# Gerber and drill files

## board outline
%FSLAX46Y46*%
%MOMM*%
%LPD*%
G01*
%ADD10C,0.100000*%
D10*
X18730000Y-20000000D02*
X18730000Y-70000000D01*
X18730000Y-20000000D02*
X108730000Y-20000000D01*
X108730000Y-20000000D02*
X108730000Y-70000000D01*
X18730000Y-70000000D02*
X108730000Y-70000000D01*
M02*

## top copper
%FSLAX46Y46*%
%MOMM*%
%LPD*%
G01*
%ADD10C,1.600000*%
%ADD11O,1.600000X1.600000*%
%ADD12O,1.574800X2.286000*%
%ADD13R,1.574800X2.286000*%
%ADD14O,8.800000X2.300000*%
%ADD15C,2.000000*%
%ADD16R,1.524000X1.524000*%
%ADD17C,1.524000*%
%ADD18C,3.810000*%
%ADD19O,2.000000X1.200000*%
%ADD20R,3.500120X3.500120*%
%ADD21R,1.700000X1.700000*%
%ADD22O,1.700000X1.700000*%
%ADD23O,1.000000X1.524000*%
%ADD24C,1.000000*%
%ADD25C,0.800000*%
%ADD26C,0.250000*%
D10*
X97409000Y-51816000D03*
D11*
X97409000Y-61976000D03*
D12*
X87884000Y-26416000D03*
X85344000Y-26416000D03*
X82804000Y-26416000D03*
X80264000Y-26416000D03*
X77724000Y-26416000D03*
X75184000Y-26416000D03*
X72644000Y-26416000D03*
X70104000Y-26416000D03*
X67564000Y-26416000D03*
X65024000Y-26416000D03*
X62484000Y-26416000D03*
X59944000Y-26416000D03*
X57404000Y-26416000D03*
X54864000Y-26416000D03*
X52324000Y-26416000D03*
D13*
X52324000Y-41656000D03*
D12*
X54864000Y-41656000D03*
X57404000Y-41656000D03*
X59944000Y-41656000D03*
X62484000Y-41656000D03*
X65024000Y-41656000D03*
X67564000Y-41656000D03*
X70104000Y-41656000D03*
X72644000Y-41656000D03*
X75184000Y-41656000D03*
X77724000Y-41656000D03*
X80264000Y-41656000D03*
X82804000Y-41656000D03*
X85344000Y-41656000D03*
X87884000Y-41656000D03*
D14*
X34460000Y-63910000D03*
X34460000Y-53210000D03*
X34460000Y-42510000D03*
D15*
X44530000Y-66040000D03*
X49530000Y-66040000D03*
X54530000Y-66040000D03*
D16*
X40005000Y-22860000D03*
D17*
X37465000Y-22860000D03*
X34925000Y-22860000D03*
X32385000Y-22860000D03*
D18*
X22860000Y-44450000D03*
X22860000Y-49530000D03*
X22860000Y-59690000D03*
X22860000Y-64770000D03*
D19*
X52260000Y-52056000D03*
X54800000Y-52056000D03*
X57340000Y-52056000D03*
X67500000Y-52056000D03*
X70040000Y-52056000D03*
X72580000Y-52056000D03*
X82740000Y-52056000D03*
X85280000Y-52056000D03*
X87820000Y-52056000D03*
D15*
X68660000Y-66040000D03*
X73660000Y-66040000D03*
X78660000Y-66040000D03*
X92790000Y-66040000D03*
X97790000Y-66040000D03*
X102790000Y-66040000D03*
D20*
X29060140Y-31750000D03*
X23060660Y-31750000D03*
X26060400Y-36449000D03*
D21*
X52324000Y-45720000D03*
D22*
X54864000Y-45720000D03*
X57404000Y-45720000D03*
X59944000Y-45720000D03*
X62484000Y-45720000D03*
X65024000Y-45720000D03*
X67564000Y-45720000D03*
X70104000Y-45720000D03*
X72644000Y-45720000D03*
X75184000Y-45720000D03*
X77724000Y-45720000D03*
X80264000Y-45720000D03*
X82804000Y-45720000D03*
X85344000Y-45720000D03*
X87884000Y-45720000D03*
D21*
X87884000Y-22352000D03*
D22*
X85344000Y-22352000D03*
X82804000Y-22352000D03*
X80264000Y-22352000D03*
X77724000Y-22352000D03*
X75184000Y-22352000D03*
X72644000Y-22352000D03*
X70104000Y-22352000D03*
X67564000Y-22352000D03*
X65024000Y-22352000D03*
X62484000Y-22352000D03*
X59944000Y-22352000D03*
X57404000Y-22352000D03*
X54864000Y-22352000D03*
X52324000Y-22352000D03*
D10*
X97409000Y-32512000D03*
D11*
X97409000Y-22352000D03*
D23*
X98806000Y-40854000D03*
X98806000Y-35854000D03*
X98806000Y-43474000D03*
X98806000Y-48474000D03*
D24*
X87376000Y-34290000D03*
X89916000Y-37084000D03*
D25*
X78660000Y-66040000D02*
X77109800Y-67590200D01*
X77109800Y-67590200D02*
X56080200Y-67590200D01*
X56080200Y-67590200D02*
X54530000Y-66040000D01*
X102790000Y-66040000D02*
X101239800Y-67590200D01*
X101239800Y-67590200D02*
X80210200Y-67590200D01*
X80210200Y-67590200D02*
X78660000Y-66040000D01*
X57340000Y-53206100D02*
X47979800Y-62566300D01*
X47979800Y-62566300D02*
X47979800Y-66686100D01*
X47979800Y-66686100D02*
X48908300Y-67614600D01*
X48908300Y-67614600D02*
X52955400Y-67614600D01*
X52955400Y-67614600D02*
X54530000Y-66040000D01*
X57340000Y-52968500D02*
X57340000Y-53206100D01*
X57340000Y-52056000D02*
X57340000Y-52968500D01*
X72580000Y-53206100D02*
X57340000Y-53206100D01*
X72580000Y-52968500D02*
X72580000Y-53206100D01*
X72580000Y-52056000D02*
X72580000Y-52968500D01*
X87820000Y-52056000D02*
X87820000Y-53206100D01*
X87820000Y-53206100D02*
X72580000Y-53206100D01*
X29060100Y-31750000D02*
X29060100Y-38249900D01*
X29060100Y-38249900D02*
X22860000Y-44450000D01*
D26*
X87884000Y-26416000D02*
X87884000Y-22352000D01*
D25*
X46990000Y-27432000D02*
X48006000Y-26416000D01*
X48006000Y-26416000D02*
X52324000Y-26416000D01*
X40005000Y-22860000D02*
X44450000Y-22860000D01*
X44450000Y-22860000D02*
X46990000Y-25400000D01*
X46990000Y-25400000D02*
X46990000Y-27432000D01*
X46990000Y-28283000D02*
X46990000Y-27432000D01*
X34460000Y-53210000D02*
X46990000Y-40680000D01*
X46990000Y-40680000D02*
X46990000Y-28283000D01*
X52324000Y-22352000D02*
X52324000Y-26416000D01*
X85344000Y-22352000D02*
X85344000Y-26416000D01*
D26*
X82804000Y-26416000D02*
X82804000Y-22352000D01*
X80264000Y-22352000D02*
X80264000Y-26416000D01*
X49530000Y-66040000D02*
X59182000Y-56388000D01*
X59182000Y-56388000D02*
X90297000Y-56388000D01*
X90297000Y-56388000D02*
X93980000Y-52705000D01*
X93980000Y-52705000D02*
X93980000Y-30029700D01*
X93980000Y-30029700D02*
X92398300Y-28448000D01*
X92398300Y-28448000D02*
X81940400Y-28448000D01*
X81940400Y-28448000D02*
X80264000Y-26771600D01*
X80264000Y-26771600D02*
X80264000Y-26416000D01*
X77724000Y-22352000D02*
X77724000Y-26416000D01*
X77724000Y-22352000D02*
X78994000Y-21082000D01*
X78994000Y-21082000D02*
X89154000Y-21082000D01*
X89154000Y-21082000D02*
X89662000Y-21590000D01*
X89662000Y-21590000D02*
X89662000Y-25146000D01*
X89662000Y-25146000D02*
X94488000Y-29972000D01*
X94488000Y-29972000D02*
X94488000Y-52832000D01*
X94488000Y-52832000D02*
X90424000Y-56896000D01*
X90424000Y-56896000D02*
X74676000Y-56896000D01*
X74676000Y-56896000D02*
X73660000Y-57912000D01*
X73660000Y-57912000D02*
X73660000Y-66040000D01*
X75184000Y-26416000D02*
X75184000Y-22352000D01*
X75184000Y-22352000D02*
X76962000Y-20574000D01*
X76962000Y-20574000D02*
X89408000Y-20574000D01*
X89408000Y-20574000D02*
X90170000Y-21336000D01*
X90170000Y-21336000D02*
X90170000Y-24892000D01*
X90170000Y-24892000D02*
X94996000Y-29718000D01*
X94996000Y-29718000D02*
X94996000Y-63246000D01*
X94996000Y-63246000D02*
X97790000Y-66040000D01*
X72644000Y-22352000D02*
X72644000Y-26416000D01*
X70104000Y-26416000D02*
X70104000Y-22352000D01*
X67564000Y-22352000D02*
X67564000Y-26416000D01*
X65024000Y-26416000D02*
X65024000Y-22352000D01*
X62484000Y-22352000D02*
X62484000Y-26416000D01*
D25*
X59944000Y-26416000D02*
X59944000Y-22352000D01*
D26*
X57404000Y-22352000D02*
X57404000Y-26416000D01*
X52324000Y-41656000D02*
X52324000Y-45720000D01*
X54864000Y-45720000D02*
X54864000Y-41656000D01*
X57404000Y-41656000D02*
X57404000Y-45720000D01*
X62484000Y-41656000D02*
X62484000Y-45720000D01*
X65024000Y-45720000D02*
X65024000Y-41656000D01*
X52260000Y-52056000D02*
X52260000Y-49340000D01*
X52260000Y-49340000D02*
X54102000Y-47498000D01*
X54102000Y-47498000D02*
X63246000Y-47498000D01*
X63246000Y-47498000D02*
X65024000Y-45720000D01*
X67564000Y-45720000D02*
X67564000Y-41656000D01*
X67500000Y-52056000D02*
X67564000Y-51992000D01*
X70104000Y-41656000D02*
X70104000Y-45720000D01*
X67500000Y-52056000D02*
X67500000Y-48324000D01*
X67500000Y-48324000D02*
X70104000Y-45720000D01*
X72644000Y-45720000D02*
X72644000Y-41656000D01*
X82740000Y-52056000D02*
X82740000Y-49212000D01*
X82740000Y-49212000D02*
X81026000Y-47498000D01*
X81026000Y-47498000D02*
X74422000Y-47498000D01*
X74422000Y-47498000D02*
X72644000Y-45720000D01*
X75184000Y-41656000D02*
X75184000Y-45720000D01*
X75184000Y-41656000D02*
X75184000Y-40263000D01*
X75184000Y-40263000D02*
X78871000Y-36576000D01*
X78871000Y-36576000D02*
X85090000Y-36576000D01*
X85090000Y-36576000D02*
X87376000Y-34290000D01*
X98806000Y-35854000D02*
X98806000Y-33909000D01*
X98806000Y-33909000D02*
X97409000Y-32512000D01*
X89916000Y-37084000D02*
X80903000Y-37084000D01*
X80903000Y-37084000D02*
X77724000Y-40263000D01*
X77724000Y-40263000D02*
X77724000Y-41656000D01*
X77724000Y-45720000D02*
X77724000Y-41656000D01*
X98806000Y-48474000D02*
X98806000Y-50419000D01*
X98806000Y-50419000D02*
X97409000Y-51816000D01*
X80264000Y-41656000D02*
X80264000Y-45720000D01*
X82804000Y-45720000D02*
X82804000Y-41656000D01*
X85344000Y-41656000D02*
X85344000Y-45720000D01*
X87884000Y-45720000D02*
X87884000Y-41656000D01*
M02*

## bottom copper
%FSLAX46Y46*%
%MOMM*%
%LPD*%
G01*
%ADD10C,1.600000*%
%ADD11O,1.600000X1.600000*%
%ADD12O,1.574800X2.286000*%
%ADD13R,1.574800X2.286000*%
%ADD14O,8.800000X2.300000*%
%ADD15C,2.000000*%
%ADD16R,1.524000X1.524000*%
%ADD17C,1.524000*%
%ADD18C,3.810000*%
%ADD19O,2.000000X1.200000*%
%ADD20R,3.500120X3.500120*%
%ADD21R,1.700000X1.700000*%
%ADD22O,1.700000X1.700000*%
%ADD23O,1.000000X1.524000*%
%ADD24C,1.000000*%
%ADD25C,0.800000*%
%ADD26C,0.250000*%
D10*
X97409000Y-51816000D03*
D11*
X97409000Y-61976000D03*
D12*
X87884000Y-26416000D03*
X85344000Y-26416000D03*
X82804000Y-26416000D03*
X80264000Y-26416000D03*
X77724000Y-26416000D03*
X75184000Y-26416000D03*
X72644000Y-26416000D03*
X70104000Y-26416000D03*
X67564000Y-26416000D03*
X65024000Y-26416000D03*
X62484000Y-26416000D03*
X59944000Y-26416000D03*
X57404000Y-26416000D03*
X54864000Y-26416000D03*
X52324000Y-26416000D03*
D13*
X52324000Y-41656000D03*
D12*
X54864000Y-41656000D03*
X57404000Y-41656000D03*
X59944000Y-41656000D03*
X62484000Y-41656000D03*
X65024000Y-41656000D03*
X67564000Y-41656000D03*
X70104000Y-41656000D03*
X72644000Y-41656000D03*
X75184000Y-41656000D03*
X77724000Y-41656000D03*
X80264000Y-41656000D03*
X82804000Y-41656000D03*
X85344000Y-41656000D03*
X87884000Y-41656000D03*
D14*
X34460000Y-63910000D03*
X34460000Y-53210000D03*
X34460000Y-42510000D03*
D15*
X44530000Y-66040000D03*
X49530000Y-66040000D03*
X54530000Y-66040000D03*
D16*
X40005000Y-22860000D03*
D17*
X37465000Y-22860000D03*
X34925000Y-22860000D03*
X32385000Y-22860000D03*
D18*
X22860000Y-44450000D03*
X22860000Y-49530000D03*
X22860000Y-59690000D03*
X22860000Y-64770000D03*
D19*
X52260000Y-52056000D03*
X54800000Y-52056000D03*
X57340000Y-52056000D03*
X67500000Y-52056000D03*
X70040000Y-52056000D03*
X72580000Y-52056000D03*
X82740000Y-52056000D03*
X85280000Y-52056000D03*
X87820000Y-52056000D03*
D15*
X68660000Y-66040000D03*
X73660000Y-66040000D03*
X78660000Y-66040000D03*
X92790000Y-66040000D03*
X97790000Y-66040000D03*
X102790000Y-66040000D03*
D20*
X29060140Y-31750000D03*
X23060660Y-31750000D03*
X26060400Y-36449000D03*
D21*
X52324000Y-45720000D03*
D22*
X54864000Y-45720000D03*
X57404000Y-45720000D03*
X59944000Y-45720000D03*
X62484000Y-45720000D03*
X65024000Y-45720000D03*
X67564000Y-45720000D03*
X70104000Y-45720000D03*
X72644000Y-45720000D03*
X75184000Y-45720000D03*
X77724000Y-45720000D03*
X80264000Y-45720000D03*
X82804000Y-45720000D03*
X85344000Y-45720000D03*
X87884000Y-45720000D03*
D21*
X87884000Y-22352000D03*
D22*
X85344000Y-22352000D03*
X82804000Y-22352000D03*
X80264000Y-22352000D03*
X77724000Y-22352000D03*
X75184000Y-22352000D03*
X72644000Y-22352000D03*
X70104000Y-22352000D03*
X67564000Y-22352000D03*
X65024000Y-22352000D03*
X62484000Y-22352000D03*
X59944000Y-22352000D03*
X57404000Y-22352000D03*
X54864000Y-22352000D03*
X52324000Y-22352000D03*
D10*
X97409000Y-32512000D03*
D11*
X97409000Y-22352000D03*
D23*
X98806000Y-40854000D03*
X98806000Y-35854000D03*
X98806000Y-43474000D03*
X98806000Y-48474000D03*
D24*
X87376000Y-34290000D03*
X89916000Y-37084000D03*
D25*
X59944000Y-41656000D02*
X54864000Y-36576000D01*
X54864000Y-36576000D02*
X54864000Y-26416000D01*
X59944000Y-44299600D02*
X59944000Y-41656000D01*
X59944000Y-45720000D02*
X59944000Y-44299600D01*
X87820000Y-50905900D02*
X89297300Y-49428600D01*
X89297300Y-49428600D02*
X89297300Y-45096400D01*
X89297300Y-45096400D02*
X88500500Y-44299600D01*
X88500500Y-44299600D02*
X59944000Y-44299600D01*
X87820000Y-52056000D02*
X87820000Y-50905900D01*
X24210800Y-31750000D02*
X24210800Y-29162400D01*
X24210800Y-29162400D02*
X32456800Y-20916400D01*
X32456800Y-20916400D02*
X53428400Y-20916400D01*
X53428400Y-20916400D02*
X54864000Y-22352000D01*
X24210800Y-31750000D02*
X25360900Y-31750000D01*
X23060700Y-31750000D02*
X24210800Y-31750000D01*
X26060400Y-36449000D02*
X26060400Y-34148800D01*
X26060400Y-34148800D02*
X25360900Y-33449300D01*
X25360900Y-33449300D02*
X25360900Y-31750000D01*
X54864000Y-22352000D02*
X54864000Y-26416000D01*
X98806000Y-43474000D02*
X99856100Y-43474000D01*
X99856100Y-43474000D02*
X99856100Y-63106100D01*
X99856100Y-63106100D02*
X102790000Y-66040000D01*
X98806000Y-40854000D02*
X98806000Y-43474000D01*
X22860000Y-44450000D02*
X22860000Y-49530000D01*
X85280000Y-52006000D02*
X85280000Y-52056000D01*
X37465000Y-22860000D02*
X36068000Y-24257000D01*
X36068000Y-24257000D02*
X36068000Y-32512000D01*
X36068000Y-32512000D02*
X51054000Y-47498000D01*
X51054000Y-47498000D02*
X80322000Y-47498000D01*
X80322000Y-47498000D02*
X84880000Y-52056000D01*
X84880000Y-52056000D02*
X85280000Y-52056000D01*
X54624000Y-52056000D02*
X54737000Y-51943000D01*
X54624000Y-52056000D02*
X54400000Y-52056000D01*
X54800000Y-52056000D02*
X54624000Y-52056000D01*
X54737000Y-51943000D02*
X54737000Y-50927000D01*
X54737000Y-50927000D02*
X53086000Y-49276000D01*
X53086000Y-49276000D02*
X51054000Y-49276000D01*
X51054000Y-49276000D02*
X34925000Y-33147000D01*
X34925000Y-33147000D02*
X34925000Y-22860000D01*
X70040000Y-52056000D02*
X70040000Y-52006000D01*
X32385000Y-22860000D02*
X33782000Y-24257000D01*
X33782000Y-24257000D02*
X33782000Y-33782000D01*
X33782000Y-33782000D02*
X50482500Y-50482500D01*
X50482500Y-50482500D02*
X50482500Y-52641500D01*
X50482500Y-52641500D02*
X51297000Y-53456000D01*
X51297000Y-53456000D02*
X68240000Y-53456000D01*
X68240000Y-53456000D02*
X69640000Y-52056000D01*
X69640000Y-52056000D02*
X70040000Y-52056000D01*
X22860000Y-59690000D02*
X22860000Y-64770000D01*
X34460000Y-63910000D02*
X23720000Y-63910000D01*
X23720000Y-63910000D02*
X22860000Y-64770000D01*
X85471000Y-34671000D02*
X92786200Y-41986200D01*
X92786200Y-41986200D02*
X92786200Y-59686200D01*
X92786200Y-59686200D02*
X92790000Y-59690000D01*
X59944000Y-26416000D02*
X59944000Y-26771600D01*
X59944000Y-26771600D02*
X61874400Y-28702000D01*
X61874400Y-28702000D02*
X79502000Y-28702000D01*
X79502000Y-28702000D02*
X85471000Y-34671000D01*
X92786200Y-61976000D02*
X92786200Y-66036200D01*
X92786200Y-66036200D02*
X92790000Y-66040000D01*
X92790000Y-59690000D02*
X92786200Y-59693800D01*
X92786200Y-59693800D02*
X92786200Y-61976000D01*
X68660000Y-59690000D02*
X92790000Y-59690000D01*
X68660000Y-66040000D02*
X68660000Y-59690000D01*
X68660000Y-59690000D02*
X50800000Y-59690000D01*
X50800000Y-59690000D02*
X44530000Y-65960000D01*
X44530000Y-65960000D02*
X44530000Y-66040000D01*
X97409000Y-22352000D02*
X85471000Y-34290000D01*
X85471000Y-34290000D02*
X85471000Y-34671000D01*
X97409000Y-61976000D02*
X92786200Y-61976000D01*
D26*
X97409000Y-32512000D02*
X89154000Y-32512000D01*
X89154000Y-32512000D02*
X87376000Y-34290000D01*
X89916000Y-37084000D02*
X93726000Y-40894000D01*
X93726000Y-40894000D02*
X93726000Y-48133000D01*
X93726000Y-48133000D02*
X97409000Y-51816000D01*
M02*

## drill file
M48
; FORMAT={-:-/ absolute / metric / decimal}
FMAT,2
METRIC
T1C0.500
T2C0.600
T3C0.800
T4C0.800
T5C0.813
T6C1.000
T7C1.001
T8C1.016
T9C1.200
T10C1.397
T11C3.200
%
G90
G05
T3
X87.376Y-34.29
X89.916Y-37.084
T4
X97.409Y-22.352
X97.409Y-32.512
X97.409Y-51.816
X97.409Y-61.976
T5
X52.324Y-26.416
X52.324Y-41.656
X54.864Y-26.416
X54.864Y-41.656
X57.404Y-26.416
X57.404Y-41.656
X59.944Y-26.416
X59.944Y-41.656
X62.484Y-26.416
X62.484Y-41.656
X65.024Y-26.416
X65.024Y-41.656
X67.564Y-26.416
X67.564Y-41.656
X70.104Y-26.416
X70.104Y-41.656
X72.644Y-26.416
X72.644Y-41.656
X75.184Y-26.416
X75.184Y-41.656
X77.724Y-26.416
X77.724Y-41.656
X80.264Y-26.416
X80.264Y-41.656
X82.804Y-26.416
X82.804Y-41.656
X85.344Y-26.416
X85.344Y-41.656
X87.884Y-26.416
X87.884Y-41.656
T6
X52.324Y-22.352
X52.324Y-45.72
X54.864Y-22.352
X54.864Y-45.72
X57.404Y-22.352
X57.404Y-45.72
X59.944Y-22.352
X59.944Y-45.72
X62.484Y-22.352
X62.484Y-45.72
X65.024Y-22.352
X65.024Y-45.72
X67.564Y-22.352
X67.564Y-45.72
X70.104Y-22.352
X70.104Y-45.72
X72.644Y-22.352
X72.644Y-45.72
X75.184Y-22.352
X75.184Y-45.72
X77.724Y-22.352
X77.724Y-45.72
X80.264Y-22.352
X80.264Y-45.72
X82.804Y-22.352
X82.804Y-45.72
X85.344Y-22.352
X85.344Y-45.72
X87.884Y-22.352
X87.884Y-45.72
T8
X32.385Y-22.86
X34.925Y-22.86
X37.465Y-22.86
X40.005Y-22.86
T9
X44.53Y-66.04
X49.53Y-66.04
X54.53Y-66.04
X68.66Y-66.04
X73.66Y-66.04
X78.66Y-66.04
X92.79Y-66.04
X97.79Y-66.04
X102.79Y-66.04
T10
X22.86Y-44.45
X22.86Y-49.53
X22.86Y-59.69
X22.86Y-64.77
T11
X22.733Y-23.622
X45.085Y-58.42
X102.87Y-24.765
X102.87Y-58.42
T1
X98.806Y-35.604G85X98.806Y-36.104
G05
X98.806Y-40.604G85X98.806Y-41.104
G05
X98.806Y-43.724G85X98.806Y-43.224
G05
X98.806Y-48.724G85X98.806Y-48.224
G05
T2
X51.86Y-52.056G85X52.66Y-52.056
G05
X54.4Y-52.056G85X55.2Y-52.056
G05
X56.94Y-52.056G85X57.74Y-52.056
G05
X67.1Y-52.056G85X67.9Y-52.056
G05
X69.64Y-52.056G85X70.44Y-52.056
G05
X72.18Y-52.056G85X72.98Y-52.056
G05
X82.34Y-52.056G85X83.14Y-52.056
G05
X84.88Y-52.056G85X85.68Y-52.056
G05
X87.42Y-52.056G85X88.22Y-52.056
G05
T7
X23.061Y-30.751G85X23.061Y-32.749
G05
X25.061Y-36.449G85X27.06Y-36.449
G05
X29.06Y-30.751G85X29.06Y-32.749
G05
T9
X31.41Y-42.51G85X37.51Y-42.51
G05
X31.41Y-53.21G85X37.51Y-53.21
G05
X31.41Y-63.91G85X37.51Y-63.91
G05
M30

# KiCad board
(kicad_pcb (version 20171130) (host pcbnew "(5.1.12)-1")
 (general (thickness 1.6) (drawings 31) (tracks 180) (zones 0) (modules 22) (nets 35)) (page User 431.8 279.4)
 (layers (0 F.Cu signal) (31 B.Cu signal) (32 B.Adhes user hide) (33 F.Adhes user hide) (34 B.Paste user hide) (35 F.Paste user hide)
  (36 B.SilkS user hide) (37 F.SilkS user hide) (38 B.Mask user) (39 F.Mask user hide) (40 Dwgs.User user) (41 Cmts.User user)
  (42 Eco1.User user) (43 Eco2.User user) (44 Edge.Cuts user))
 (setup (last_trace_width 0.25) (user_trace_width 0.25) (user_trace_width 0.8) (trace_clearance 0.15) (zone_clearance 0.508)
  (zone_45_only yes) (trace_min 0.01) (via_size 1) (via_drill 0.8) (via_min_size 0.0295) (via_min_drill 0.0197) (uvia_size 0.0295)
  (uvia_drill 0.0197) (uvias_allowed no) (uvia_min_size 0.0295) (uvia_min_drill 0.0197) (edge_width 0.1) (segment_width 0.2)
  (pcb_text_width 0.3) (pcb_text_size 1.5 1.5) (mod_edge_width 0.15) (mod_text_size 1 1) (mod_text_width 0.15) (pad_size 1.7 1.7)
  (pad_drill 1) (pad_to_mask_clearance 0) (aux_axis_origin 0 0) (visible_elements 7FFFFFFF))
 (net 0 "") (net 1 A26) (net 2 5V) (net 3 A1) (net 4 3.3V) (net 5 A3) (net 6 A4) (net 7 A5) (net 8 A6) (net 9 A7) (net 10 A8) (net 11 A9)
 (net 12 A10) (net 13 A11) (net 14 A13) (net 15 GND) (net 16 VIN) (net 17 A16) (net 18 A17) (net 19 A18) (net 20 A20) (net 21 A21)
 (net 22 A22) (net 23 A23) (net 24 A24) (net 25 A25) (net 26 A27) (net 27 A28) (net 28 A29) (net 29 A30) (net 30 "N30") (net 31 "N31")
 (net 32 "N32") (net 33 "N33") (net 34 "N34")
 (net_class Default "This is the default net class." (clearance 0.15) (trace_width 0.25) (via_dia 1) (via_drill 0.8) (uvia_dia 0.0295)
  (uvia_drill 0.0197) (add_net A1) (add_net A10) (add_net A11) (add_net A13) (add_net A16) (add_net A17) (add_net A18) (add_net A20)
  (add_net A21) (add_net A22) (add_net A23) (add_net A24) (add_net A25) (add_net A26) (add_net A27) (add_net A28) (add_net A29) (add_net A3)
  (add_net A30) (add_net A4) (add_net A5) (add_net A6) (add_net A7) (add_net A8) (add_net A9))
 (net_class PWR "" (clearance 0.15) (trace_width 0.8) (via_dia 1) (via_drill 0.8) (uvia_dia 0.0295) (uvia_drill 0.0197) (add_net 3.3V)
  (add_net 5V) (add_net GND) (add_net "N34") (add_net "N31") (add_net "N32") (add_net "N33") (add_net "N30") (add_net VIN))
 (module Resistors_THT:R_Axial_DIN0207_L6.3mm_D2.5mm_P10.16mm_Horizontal (layer F.Cu) (at 97.409 51.816 270)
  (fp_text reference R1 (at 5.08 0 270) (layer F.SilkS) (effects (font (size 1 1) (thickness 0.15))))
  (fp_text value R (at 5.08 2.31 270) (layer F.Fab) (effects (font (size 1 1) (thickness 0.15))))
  (pad 1 thru_hole circle (at 0 0 270) (size 1.6 1.6) (drill 0.8) (layers *.Cu *.Mask) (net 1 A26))
  (pad 2 thru_hole oval (at 10.16 0 270) (size 1.6 1.6) (drill 0.8) (layers *.Cu *.Mask) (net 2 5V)))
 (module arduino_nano (layer F.Cu) (at 68.834 34.036 180)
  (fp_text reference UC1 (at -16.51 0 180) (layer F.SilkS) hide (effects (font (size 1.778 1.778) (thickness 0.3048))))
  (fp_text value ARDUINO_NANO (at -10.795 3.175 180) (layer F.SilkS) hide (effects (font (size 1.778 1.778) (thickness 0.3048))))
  (pad 1 thru_hole oval (at -19.05 7.62 180) (size 1.5748 2.286) (drill 0.8128) (layers *.Cu *.Mask F.SilkS) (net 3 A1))
  (pad 2 thru_hole oval (at -16.51 7.62 180) (size 1.5748 2.286) (drill 0.8128) (layers *.Cu *.Mask F.SilkS) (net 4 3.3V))
  (pad 3 thru_hole oval (at -13.97 7.62 180) (size 1.5748 2.286) (drill 0.8128) (layers *.Cu *.Mask F.SilkS) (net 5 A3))
  (pad 4 thru_hole oval (at -11.43 7.62 180) (size 1.5748 2.286) (drill 0.8128) (layers *.Cu *.Mask F.SilkS) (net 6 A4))
  (pad 5 thru_hole oval (at -8.89 7.62 180) (size 1.5748 2.286) (drill 0.8128) (layers *.Cu *.Mask F.SilkS) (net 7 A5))
  (pad 6 thru_hole oval (at -6.35 7.62 180) (size 1.5748 2.286) (drill 0.8128) (layers *.Cu *.Mask F.SilkS) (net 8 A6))
  (pad 7 thru_hole oval (at -3.81 7.62 180) (size 1.5748 2.286) (drill 0.8128) (layers *.Cu *.Mask F.SilkS) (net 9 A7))
  (pad 8 thru_hole oval (at -1.27 7.62 180) (size 1.5748 2.286) (drill 0.8128) (layers *.Cu *.Mask F.SilkS) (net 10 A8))
  (pad 9 thru_hole oval (at 1.27 7.62 180) (size 1.5748 2.286) (drill 0.8128) (layers *.Cu *.Mask F.SilkS) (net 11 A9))
  (pad 10 thru_hole oval (at 3.81 7.62 180) (size 1.5748 2.286) (drill 0.8128) (layers *.Cu *.Mask F.SilkS) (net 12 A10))
  (pad 11 thru_hole oval (at 6.35 7.62 180) (size 1.5748 2.286) (drill 0.8128) (layers *.Cu *.Mask F.SilkS) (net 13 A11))
  (pad 12 thru_hole oval (at 8.89 7.62 180) (size 1.5748 2.286) (drill 0.8128) (layers *.Cu *.Mask F.SilkS) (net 2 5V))
  (pad 13 thru_hole oval (at 11.43 7.62 180) (size 1.5748 2.286) (drill 0.8128) (layers *.Cu *.Mask F.SilkS) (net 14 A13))
  (pad 14 thru_hole oval (at 13.97 7.62 180) (size 1.5748 2.286) (drill 0.8128) (layers *.Cu *.Mask F.SilkS) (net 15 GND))
  (pad 15 thru_hole oval (at 16.51 7.62 180) (size 1.5748 2.286) (drill 0.8128) (layers *.Cu *.Mask F.SilkS) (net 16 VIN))
  (pad 16 thru_hole rect (at 16.51 -7.62 180) (size 1.5748 2.286) (drill 0.8128) (layers *.Cu *.Mask F.SilkS) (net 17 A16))
  (pad 17 thru_hole oval (at 13.97 -7.62 180) (size 1.5748 2.286) (drill 0.8128) (layers *.Cu *.Mask F.SilkS) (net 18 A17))
  (pad 18 thru_hole oval (at 11.43 -7.62 180) (size 1.5748 2.286) (drill 0.8128) (layers *.Cu *.Mask F.SilkS) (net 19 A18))
  (pad 19 thru_hole oval (at 8.89 -7.62 180) (size 1.5748 2.286) (drill 0.8128) (layers *.Cu *.Mask F.SilkS) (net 15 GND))
  (pad 20 thru_hole oval (at 6.35 -7.62 180) (size 1.5748 2.286) (drill 0.8128) (layers *.Cu *.Mask F.SilkS) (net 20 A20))
  (pad 21 thru_hole oval (at 3.81 -7.62 180) (size 1.5748 2.286) (drill 0.8128) (layers *.Cu *.Mask F.SilkS) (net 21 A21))
  (pad 22 thru_hole oval (at 1.27 -7.62 180) (size 1.5748 2.286) (drill 0.8128) (layers *.Cu *.Mask F.SilkS) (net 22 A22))
  (pad 23 thru_hole oval (at -1.27 -7.62 180) (size 1.5748 2.286) (drill 0.8128) (layers *.Cu *.Mask F.SilkS) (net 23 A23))
  (pad 24 thru_hole oval (at -3.81 -7.62 180) (size 1.5748 2.286) (drill 0.8128) (layers *.Cu *.Mask F.SilkS) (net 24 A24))
  (pad 25 thru_hole oval (at -6.35 -7.62 180) (size 1.5748 2.286) (drill 0.8128) (layers *.Cu *.Mask F.SilkS) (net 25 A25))
  (pad 26 thru_hole oval (at -8.89 -7.62 180) (size 1.5748 2.286) (drill 0.8128) (layers *.Cu *.Mask F.SilkS) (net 1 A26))
  (pad 27 thru_hole oval (at -11.43 -7.62 180) (size 1.5748 2.286) (drill 0.8128) (layers *.Cu *.Mask F.SilkS) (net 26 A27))
  (pad 28 thru_hole oval (at -13.97 -7.62 180) (size 1.5748 2.286) (drill 0.8128) (layers *.Cu *.Mask F.SilkS) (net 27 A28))
  (pad 29 thru_hole oval (at -16.51 -7.62 180) (size 1.5748 2.286) (drill 0.8128) (layers *.Cu *.Mask F.SilkS) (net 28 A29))
  (pad 30 thru_hole oval (at -19.05 -7.62 180) (size 1.5748 2.286) (drill 0.8128) (layers *.Cu *.Mask F.SilkS) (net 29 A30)))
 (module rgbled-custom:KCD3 (layer F.Cu) (at 29.21 67.31 90)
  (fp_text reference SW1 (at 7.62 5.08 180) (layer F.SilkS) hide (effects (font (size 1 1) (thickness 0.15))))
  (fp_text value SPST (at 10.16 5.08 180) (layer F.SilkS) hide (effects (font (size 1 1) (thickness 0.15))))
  (pad 1 thru_hole oval (at 3.4 5.25 90) (size 2.3 8.8) (drill oval 1.2 7.3) (layers *.Cu *.Mask F.SilkS) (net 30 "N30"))
  (pad 2 thru_hole oval (at 14.1 5.25 90) (size 2.3 8.8) (drill oval 1.2 7.3) (layers *.Cu *.Mask F.SilkS) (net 16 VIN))
  (pad 3 thru_hole oval (at 24.8 5.25 90) (size 2.3 8.8) (drill oval 1.2 7.3) (layers *.Cu *.Mask F.SilkS)))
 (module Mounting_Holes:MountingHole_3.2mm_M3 (layer F.Cu) (at 22.733 23.622)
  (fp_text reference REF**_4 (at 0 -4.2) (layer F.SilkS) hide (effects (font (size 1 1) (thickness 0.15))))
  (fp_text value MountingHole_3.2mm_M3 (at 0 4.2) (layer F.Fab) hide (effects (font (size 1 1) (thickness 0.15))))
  (pad 1 np_thru_hole circle (at 0 0) (size 3.2 3.2) (drill 3.2) (layers *.Cu *.Mask F.SilkS)))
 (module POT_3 (layer F.Cu) (at 49.53 66.04)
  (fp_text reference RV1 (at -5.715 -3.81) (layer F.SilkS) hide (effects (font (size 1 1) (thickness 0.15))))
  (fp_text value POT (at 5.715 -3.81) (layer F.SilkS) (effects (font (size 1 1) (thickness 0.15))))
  (pad 1 thru_hole circle (at -5 0) (size 2 2) (drill 1.2) (layers *.Cu *.Mask F.SilkS) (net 2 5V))
  (pad 2 thru_hole circle (at 0 0) (size 2 2) (drill 1.2) (layers *.Cu *.Mask F.SilkS) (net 6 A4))
  (pad 3 thru_hole circle (at 5 0) (size 2 2) (drill 1.2) (layers *.Cu *.Mask F.SilkS) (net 15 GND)))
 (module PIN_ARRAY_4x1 (layer F.Cu) (at 36.195 22.86 180)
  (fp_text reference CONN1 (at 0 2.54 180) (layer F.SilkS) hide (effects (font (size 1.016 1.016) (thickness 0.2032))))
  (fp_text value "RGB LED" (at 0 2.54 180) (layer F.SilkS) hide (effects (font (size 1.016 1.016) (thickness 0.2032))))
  (pad 1 thru_hole rect (at -3.81 0 180) (size 1.524 1.524) (drill 1.016) (layers *.Cu *.Mask F.SilkS) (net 16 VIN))
  (pad 2 thru_hole circle (at -1.27 0 180) (size 1.524 1.524) (drill 1.016) (layers *.Cu *.Mask F.SilkS) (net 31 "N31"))
  (pad 3 thru_hole circle (at 1.27 0 180) (size 1.524 1.524) (drill 1.016) (layers *.Cu *.Mask F.SilkS) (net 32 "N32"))
  (pad 4 thru_hole circle (at 3.81 0 180) (size 1.524 1.524) (drill 1.016) (layers *.Cu *.Mask F.SilkS) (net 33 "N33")))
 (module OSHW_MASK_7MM (layer F.Cu) (at 38.481 30.099)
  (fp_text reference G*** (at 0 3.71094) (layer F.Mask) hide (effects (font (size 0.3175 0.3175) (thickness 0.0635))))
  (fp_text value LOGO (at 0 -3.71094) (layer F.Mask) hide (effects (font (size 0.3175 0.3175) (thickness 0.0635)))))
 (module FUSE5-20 (layer F.Cu) (at 22.86 54.61 270)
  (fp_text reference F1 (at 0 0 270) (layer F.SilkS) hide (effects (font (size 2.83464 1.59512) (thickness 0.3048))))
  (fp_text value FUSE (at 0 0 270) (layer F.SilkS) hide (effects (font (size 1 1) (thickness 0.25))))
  (pad 1 thru_hole circle (at -10.16 0 270) (size 3.81 3.81) (drill 1.397) (layers *.Cu *.Mask F.SilkS) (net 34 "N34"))
  (pad 1 thru_hole circle (at -5.08 0 270) (size 3.81 3.81) (drill 1.397) (layers *.Cu *.Mask F.SilkS) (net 34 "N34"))
  (pad 2 thru_hole circle (at 5.08 0 270) (size 3.81 3.81) (drill 1.397) (layers *.Cu *.Mask F.SilkS) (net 30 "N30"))
  (pad 2 thru_hole circle (at 10.16 0 270) (size 3.81 3.81) (drill 1.397) (layers *.Cu *.Mask F.SilkS) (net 30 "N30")))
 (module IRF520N (layer F.Cu) (at 49.53 49.276)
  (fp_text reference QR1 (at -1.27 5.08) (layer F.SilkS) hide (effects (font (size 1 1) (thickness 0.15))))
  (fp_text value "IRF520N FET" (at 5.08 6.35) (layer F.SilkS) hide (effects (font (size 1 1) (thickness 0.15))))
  (pad G thru_hole oval (at 2.73 2.78) (size 2 1.2) (drill oval 1.4 0.6) (layers *.Cu *.Mask F.SilkS) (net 21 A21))
  (pad D thru_hole oval (at 5.27 2.78) (size 2 1.2) (drill oval 1.4 0.6) (layers *.Cu *.Mask F.SilkS) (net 32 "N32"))
  (pad S thru_hole oval (at 7.81 2.78) (size 2 1.2) (drill oval 1.4 0.6) (layers *.Cu *.Mask F.SilkS) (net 15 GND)))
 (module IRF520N (layer F.Cu) (at 64.77 49.276)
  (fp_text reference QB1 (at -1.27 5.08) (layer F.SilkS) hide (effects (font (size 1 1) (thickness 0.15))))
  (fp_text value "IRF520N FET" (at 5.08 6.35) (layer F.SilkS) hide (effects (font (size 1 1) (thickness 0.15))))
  (pad G thru_hole oval (at 2.73 2.78) (size 2 1.2) (drill oval 1.4 0.6) (layers *.Cu *.Mask F.SilkS) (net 23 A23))
  (pad D thru_hole oval (at 5.27 2.78) (size 2 1.2) (drill oval 1.4 0.6) (layers *.Cu *.Mask F.SilkS) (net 33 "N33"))
  (pad S thru_hole oval (at 7.81 2.78) (size 2 1.2) (drill oval 1.4 0.6) (layers *.Cu *.Mask F.SilkS) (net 15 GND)))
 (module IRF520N (layer F.Cu) (at 80.01 49.276)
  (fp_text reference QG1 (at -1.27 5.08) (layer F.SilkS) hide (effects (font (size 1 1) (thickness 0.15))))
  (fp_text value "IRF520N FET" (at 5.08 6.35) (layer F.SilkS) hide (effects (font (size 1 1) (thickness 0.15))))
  (pad G thru_hole oval (at 2.73 2.78) (size 2 1.2) (drill oval 1.4 0.6) (layers *.Cu *.Mask F.SilkS) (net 24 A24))
  (pad D thru_hole oval (at 5.27 2.78) (size 2 1.2) (drill oval 1.4 0.6) (layers *.Cu *.Mask F.SilkS) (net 31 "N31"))
  (pad S thru_hole oval (at 7.81 2.78) (size 2 1.2) (drill oval 1.4 0.6) (layers *.Cu *.Mask F.SilkS) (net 15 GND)))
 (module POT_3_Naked (layer F.Cu) (at 73.66 66.04)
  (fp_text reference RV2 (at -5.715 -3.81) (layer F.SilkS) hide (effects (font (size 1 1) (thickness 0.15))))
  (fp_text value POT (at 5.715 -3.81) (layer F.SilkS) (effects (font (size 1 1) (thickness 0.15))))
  (pad 1 thru_hole circle (at -5 0) (size 2 2) (drill 1.2) (layers *.Cu *.Mask F.SilkS) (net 2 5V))
  (pad 2 thru_hole circle (at 0 0) (size 2 2) (drill 1.2) (layers *.Cu *.Mask F.SilkS) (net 7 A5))
  (pad 3 thru_hole circle (at 5 0) (size 2 2) (drill 1.2) (layers *.Cu *.Mask F.SilkS) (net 15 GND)))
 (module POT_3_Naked (layer F.Cu) (at 97.79 66.04)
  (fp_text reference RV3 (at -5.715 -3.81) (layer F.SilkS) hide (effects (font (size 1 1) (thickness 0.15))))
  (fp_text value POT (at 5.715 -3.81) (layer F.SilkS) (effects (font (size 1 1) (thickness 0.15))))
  (pad 1 thru_hole circle (at -5 0) (size 2 2) (drill 1.2) (layers *.Cu *.Mask F.SilkS) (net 2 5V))
  (pad 2 thru_hole circle (at 0 0) (size 2 2) (drill 1.2) (layers *.Cu *.Mask F.SilkS) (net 8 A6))
  (pad 3 thru_hole circle (at 5 0) (size 2 2) (drill 1.2) (layers *.Cu *.Mask F.SilkS) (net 15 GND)))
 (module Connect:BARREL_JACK (layer F.Cu) (at 22.86 31.75)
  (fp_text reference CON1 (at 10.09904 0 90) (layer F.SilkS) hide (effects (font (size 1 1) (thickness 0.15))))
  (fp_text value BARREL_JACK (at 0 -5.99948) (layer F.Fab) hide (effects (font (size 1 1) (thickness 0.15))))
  (pad 1 thru_hole rect (at 6.20014 0) (size 3.50012 3.50012) (drill oval 1.00076 2.99974) (layers *.Cu *.Mask F.SilkS) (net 34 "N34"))
  (pad 2 thru_hole rect (at 0.20066 0) (size 3.50012 3.50012) (drill oval 1.00076 2.99974) (layers *.Cu *.Mask F.SilkS) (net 15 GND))
  (pad 3 thru_hole rect (at 3.2004 4.699) (size 3.50012 3.50012) (drill oval 2.99974 1.00076) (layers *.Cu *.Mask F.SilkS) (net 15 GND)))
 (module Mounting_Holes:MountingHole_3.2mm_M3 (layer F.Cu) (at 102.87 24.765)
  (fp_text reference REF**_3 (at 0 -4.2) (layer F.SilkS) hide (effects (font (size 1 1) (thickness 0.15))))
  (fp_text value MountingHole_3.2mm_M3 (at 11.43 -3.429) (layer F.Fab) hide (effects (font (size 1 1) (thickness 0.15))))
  (pad 1 np_thru_hole circle (at 0 0) (size 3.2 3.2) (drill 3.2) (layers *.Cu *.Mask F.SilkS)))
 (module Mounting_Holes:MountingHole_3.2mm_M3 (layer F.Cu) (at 45.085 58.42)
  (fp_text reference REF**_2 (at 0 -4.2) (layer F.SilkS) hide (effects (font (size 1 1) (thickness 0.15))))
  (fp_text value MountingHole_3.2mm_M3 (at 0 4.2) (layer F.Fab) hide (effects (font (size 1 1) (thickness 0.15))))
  (pad 1 np_thru_hole circle (at 0 0) (size 3.2 3.2) (drill 3.2) (layers *.Cu *.Mask F.SilkS)))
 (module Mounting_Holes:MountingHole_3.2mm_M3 (layer F.Cu) (at 102.87 58.42)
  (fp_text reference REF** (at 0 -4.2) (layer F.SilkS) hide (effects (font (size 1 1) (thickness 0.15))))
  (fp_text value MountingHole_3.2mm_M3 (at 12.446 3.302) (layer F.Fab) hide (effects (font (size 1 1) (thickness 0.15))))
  (pad 1 np_thru_hole circle (at 0 0) (size 3.2 3.2) (drill 3.2) (layers *.Cu *.Mask F.SilkS)))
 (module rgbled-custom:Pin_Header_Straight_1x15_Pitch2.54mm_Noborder (layer F.Cu) (at 52.324 45.72 90)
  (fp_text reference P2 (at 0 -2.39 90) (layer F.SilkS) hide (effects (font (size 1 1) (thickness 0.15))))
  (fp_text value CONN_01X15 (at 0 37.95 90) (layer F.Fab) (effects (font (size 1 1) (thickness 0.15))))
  (pad 1 thru_hole rect (at 0 0 90) (size 1.7 1.7) (drill 1) (layers *.Cu *.Mask) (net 17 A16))
  (pad 2 thru_hole oval (at 0 2.54 90) (size 1.7 1.7) (drill 1) (layers *.Cu *.Mask) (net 18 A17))
  (pad 3 thru_hole oval (at 0 5.08 90) (size 1.7 1.7) (drill 1) (layers *.Cu *.Mask) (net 19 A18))
  (pad 4 thru_hole oval (at 0 7.62 90) (size 1.7 1.7) (drill 1) (layers *.Cu *.Mask) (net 15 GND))
  (pad 5 thru_hole oval (at 0 10.16 90) (size 1.7 1.7) (drill 1) (layers *.Cu *.Mask) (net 20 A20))
  (pad 6 thru_hole oval (at 0 12.7 90) (size 1.7 1.7) (drill 1) (layers *.Cu *.Mask) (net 21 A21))
  (pad 7 thru_hole oval (at 0 15.24 90) (size 1.7 1.7) (drill 1) (layers *.Cu *.Mask) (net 22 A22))
  (pad 8 thru_hole oval (at 0 17.78 90) (size 1.7 1.7) (drill 1) (layers *.Cu *.Mask) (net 23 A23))
  (pad 9 thru_hole oval (at 0 20.32 90) (size 1.7 1.7) (drill 1) (layers *.Cu *.Mask) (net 24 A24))
  (pad 10 thru_hole oval (at 0 22.86 90) (size 1.7 1.7) (drill 1) (layers *.Cu *.Mask) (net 25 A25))
  (pad 11 thru_hole oval (at 0 25.4 90) (size 1.7 1.7) (drill 1) (layers *.Cu *.Mask) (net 1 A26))
  (pad 12 thru_hole oval (at 0 27.94 90) (size 1.7 1.7) (drill 1) (layers *.Cu *.Mask) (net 26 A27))
  (pad 13 thru_hole oval (at 0 30.48 90) (size 1.7 1.7) (drill 1) (layers *.Cu *.Mask) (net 27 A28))
  (pad 14 thru_hole oval (at 0 33.02 90) (size 1.7 1.7) (drill 1) (layers *.Cu *.Mask) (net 28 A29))
  (pad 15 thru_hole oval (at 0 35.56 90) (size 1.7 1.7) (drill 1) (layers *.Cu *.Mask) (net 29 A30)))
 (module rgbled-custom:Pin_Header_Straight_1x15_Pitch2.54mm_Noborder (layer F.Cu) (at 87.884 22.352 270)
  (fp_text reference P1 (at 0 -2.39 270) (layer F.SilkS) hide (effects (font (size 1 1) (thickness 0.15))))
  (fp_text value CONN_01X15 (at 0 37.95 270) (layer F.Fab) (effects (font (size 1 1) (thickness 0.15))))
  (pad 1 thru_hole rect (at 0 0 270) (size 1.7 1.7) (drill 1) (layers *.Cu *.Mask) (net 3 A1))
  (pad 2 thru_hole oval (at 0 2.54 270) (size 1.7 1.7) (drill 1) (layers *.Cu *.Mask) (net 4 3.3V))
  (pad 3 thru_hole oval (at 0 5.08 270) (size 1.7 1.7) (drill 1) (layers *.Cu *.Mask) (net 5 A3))
  (pad 4 thru_hole oval (at 0 7.62 270) (size 1.7 1.7) (drill 1) (layers *.Cu *.Mask) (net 6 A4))
  (pad 5 thru_hole oval (at 0 10.16 270) (size 1.7 1.7) (drill 1) (layers *.Cu *.Mask) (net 7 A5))
  (pad 6 thru_hole oval (at 0 12.7 270) (size 1.7 1.7) (drill 1) (layers *.Cu *.Mask) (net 8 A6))
  (pad 7 thru_hole oval (at 0 15.24 270) (size 1.7 1.7) (drill 1) (layers *.Cu *.Mask) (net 9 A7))
  (pad 8 thru_hole oval (at 0 17.78 270) (size 1.7 1.7) (drill 1) (layers *.Cu *.Mask) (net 10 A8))
  (pad 9 thru_hole oval (at 0 20.32 270) (size 1.7 1.7) (drill 1) (layers *.Cu *.Mask) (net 11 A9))
  (pad 10 thru_hole oval (at 0 22.86 270) (size 1.7 1.7) (drill 1) (layers *.Cu *.Mask) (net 12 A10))
  (pad 11 thru_hole oval (at 0 25.4 270) (size 1.7 1.7) (drill 1) (layers *.Cu *.Mask) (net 13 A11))
  (pad 12 thru_hole oval (at 0 27.94 270) (size 1.7 1.7) (drill 1) (layers *.Cu *.Mask) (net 2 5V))
  (pad 13 thru_hole oval (at 0 30.48 270) (size 1.7 1.7) (drill 1) (layers *.Cu *.Mask) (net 14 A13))
  (pad 14 thru_hole oval (at 0 33.02 270) (size 1.7 1.7) (drill 1) (layers *.Cu *.Mask) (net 15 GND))
  (pad 15 thru_hole oval (at 0 35.56 270) (size 1.7 1.7) (drill 1) (layers *.Cu *.Mask) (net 16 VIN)))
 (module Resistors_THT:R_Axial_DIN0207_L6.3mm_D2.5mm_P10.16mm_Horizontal (layer F.Cu) (at 97.409 32.512 90)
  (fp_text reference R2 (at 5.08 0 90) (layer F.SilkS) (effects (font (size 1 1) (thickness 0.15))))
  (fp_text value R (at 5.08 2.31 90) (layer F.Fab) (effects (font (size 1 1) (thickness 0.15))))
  (pad 1 thru_hole circle (at 0 0 90) (size 1.6 1.6) (drill 0.8) (layers *.Cu *.Mask) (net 25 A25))
  (pad 2 thru_hole oval (at 10.16 0 90) (size 1.6 1.6) (drill 0.8) (layers *.Cu *.Mask) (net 2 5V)))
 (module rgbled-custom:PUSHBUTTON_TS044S (layer F.Cu) (at 98.806 38.354 270)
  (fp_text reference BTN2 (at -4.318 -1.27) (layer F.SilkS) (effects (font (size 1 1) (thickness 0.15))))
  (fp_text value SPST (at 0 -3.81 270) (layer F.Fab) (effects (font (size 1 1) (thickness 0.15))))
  (pad 2 thru_hole oval (at 2.5 0 270) (size 1.524 1) (drill oval 1 0.5) (layers *.Cu *.Mask) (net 15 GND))
  (pad 1 thru_hole oval (at -2.5 0 270) (size 1.524 1) (drill oval 1 0.5) (layers *.Cu *.Mask) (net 25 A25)))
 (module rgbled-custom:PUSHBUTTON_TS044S (layer F.Cu) (at 98.806 45.974 90)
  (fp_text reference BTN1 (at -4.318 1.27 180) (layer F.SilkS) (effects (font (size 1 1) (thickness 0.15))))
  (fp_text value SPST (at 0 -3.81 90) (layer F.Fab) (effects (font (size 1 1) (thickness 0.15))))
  (pad 2 thru_hole oval (at 2.5 0 90) (size 1.524 1) (drill oval 1 0.5) (layers *.Cu *.Mask) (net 15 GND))
  (pad 1 thru_hole oval (at -2.5 0 90) (size 1.524 1) (drill oval 1 0.5) (layers *.Cu *.Mask) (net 1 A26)))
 (gr_line (start 18.73 20) (end 18.73 70) (angle 90) (layer Edge.Cuts) (width 0.1))
 (gr_line (start 18.73 20) (end 108.73 20) (angle 90) (layer Edge.Cuts) (width 0.1))
 (gr_line (start 108.73 20) (end 108.73 70) (angle 90) (layer Edge.Cuts) (width 0.1))
 (gr_line (start 18.73 70) (end 108.73 70) (angle 90) (layer Edge.Cuts) (width 0.1))
 (segment (start 59.944 41.656) (end 54.864 36.576) (width 0.8) (layer B.Cu) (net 15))
 (segment (start 54.864 36.576) (end 54.864 26.416) (width 0.8) (layer B.Cu) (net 15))
 (segment (start 59.944 44.2996) (end 59.944 41.656) (width 0.8) (layer B.Cu) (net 15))
 (segment (start 59.944 45.72) (end 59.944 44.2996) (width 0.8) (layer B.Cu) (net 15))
 (segment (start 87.82 50.9059) (end 89.2973 49.4286) (width 0.8) (layer B.Cu) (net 15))
 (segment (start 89.2973 49.4286) (end 89.2973 45.0964) (width 0.8) (layer B.Cu) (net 15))
 (segment (start 89.2973 45.0964) (end 88.5005 44.2996) (width 0.8) (layer B.Cu) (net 15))
 (segment (start 88.5005 44.2996) (end 59.944 44.2996) (width 0.8) (layer B.Cu) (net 15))
 (segment (start 87.82 52.056) (end 87.82 50.9059) (width 0.8) (layer B.Cu) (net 15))
 (segment (start 78.66 66.04) (end 77.1098 67.5902) (width 0.8) (layer F.Cu) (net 15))
 (segment (start 77.1098 67.5902) (end 56.0802 67.5902) (width 0.8) (layer F.Cu) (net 15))
 (segment (start 56.0802 67.5902) (end 54.53 66.04) (width 0.8) (layer F.Cu) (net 15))
 (segment (start 102.79 66.04) (end 101.2398 67.5902) (width 0.8) (layer F.Cu) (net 15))
 (segment (start 101.2398 67.5902) (end 80.2102 67.5902) (width 0.8) (layer F.Cu) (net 15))
 (segment (start 80.2102 67.5902) (end 78.66 66.04) (width 0.8) (layer F.Cu) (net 15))
 (segment (start 57.34 53.2061) (end 47.9798 62.5663) (width 0.8) (layer F.Cu) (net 15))
 (segment (start 47.9798 62.5663) (end 47.9798 66.6861) (width 0.8) (layer F.Cu) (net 15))
 (segment (start 47.9798 66.6861) (end 48.9083 67.6146) (width 0.8) (layer F.Cu) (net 15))
 (segment (start 48.9083 67.6146) (end 52.9554 67.6146) (width 0.8) (layer F.Cu) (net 15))
 (segment (start 52.9554 67.6146) (end 54.53 66.04) (width 0.8) (layer F.Cu) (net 15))
 (segment (start 57.34 52.9685) (end 57.34 53.2061) (width 0.8) (layer F.Cu) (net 15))
 (segment (start 57.34 52.056) (end 57.34 52.9685) (width 0.8) (layer F.Cu) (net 15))
 (segment (start 72.58 53.2061) (end 57.34 53.2061) (width 0.8) (layer F.Cu) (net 15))
 (segment (start 72.58 52.9685) (end 72.58 53.2061) (width 0.8) (layer F.Cu) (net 15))
 (segment (start 72.58 52.056) (end 72.58 52.9685) (width 0.8) (layer F.Cu) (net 15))
 (segment (start 87.82 52.056) (end 87.82 53.2061) (width 0.8) (layer F.Cu) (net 15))
 (segment (start 87.82 53.2061) (end 72.58 53.2061) (width 0.8) (layer F.Cu) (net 15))
 (segment (start 24.2108 31.75) (end 24.2108 29.1624) (width 0.8) (layer B.Cu) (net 15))
 (segment (start 24.2108 29.1624) (end 32.4568 20.9164) (width 0.8) (layer B.Cu) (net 15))
 (segment (start 32.4568 20.9164) (end 53.4284 20.9164) (width 0.8) (layer B.Cu) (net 15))
 (segment (start 53.4284 20.9164) (end 54.864 22.352) (width 0.8) (layer B.Cu) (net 15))
 (segment (start 24.2108 31.75) (end 25.3609 31.75) (width 0.8) (layer B.Cu) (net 15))
 (segment (start 23.0607 31.75) (end 24.2108 31.75) (width 0.8) (layer B.Cu) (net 15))
 (segment (start 26.0604 36.449) (end 26.0604 34.1488) (width 0.8) (layer B.Cu) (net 15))
 (segment (start 26.0604 34.1488) (end 25.3609 33.4493) (width 0.8) (layer B.Cu) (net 15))
 (segment (start 25.3609 33.4493) (end 25.3609 31.75) (width 0.8) (layer B.Cu) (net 15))
 (segment (start 54.864 22.352) (end 54.864 26.416) (width 0.8) (layer B.Cu) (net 15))
 (segment (start 98.806 43.474) (end 99.8561 43.474) (width 0.8) (layer B.Cu) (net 15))
 (segment (start 99.8561 43.474) (end 99.8561 63.1061) (width 0.8) (layer B.Cu) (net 15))
 (segment (start 99.8561 63.1061) (end 102.79 66.04) (width 0.8) (layer B.Cu) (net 15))
 (segment (start 98.806 40.854) (end 98.806 43.474) (width 0.8) (layer B.Cu) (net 15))
 (segment (start 22.86 44.45) (end 22.86 49.53) (width 0.8) (layer B.Cu) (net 34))
 (segment (start 29.0601 31.75) (end 29.0601 38.2499) (width 0.8) (layer F.Cu) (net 34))
 (segment (start 29.0601 38.2499) (end 22.86 44.45) (width 0.8) (layer F.Cu) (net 34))
 (segment (start 85.28 52.006) (end 85.28 52.056) (width 0.8) (layer B.Cu) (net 31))
 (segment (start 37.465 22.86) (end 36.068 24.257) (width 0.8) (layer B.Cu) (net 31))
 (segment (start 36.068 24.257) (end 36.068 32.512) (width 0.8) (layer B.Cu) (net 31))
 (segment (start 36.068 32.512) (end 51.054 47.498) (width 0.8) (layer B.Cu) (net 31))
 (segment (start 51.054 47.498) (end 80.322 47.498) (width 0.8) (layer B.Cu) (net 31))
 (segment (start 80.322 47.498) (end 84.88 52.056) (width 0.8) (layer B.Cu) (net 31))
 (segment (start 84.88 52.056) (end 85.28 52.056) (width 0.8) (layer B.Cu) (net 31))
 (segment (start 54.624 52.056) (end 54.737 51.943) (width 0.8) (layer B.Cu) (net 32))
 (segment (start 54.624 52.056) (end 54.4 52.056) (width 0.8) (layer B.Cu) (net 32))
 (segment (start 54.8 52.056) (end 54.624 52.056) (width 0.8) (layer B.Cu) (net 32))
 (segment (start 54.737 51.943) (end 54.737 50.927) (width 0.8) (layer B.Cu) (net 32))
 (segment (start 54.737 50.927) (end 53.086 49.276) (width 0.8) (layer B.Cu) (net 32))
 (segment (start 53.086 49.276) (end 51.054 49.276) (width 0.8) (layer B.Cu) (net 32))
 (segment (start 51.054 49.276) (end 34.925 33.147) (width 0.8) (layer B.Cu) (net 32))
 (segment (start 34.925 33.147) (end 34.925 22.86) (width 0.8) (layer B.Cu) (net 32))
 (segment (start 70.04 52.056) (end 70.04 52.006) (width 0.8) (layer B.Cu) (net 33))
 (segment (start 32.385 22.86) (end 33.782 24.257) (width 0.8) (layer B.Cu) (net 33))
 (segment (start 33.782 24.257) (end 33.782 33.782) (width 0.8) (layer B.Cu) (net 33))
 (segment (start 33.782 33.782) (end 50.4825 50.4825) (width 0.8) (layer B.Cu) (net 33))
 (segment (start 50.4825 50.4825) (end 50.4825 52.6415) (width 0.8) (layer B.Cu) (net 33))
 (segment (start 50.4825 52.6415) (end 51.297 53.456) (width 0.8) (layer B.Cu) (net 33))
 (segment (start 51.297 53.456) (end 68.24 53.456) (width 0.8) (layer B.Cu) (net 33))
 (segment (start 68.24 53.456) (end 69.64 52.056) (width 0.8) (layer B.Cu) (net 33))
 (segment (start 69.64 52.056) (end 70.04 52.056) (width 0.8) (layer B.Cu) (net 33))
 (segment (start 22.86 59.69) (end 22.86 64.77) (width 0.8) (layer B.Cu) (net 30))
 (segment (start 34.46 63.91) (end 23.72 63.91) (width 0.8) (layer B.Cu) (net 30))
 (segment (start 23.72 63.91) (end 22.86 64.77) (width 0.8) (layer B.Cu) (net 30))
 (segment (start 87.884 26.416) (end 87.884 22.352) (width 0.25) (layer F.Cu) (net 3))
 (segment (start 46.99 27.432) (end 48.006 26.416) (width 0.8) (layer F.Cu) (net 16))
 (segment (start 48.006 26.416) (end 52.324 26.416) (width 0.8) (layer F.Cu) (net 16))
 (segment (start 40.005 22.86) (end 44.45 22.86) (width 0.8) (layer F.Cu) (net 16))
 (segment (start 44.45 22.86) (end 46.99 25.4) (width 0.8) (layer F.Cu) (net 16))
 (segment (start 46.99 25.4) (end 46.99 27.432) (width 0.8) (layer F.Cu) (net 16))
 (segment (start 46.99 28.283) (end 46.99 27.432) (width 0.8) (layer F.Cu) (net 16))
 (segment (start 34.46 53.21) (end 46.99 40.68) (width 0.8) (layer F.Cu) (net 16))
 (segment (start 46.99 40.68) (end 46.99 28.283) (width 0.8) (layer F.Cu) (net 16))
 (segment (start 52.324 22.352) (end 52.324 26.416) (width 0.8) (layer F.Cu) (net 16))
 (segment (start 85.344 22.352) (end 85.344 26.416) (width 0.8) (layer F.Cu) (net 4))
 (segment (start 82.804 26.416) (end 82.804 22.352) (width 0.25) (layer F.Cu) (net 5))
 (segment (start 80.264 22.352) (end 80.264 26.416) (width 0.25) (layer F.Cu) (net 6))
 (segment (start 49.53 66.04) (end 59.182 56.388) (width 0.25) (layer F.Cu) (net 6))
 (segment (start 59.182 56.388) (end 90.297 56.388) (width 0.25) (layer F.Cu) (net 6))
 (segment (start 90.297 56.388) (end 93.98 52.705) (width 0.25) (layer F.Cu) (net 6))
 (segment (start 93.98 52.705) (end 93.98 30.0297) (width 0.25) (layer F.Cu) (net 6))
 (segment (start 93.98 30.0297) (end 92.3983 28.448) (width 0.25) (layer F.Cu) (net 6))
 (segment (start 92.3983 28.448) (end 81.9404 28.448) (width 0.25) (layer F.Cu) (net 6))
 (segment (start 81.9404 28.448) (end 80.264 26.7716) (width 0.25) (layer F.Cu) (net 6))
 (segment (start 80.264 26.7716) (end 80.264 26.416) (width 0.25) (layer F.Cu) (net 6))
 (segment (start 77.724 22.352) (end 77.724 26.416) (width 0.25) (layer F.Cu) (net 7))
 (segment (start 77.724 22.352) (end 78.994 21.082) (width 0.25) (layer F.Cu) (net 7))
 (segment (start 78.994 21.082) (end 89.154 21.082) (width 0.25) (layer F.Cu) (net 7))
 (segment (start 89.154 21.082) (end 89.662 21.59) (width 0.25) (layer F.Cu) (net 7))
 (segment (start 89.662 21.59) (end 89.662 25.146) (width 0.25) (layer F.Cu) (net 7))
 (segment (start 89.662 25.146) (end 94.488 29.972) (width 0.25) (layer F.Cu) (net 7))
 (segment (start 94.488 29.972) (end 94.488 52.832) (width 0.25) (layer F.Cu) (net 7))
 (segment (start 94.488 52.832) (end 90.424 56.896) (width 0.25) (layer F.Cu) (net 7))
 (segment (start 90.424 56.896) (end 74.676 56.896) (width 0.25) (layer F.Cu) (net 7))
 (segment (start 74.676 56.896) (end 73.66 57.912) (width 0.25) (layer F.Cu) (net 7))
 (segment (start 73.66 57.912) (end 73.66 66.04) (width 0.25) (layer F.Cu) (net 7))
 (segment (start 75.184 26.416) (end 75.184 22.352) (width 0.25) (layer F.Cu) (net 8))
 (segment (start 75.184 22.352) (end 76.962 20.574) (width 0.25) (layer F.Cu) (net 8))
 (segment (start 76.962 20.574) (end 89.408 20.574) (width 0.25) (layer F.Cu) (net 8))
 (segment (start 89.408 20.574) (end 90.17 21.336) (width 0.25) (layer F.Cu) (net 8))
 (segment (start 90.17 21.336) (end 90.17 24.892) (width 0.25) (layer F.Cu) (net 8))
 (segment (start 90.17 24.892) (end 94.996 29.718) (width 0.25) (layer F.Cu) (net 8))
 (segment (start 94.996 29.718) (end 94.996 63.246) (width 0.25) (layer F.Cu) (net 8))
 (segment (start 94.996 63.246) (end 97.79 66.04) (width 0.25) (layer F.Cu) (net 8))
 (segment (start 72.644 22.352) (end 72.644 26.416) (width 0.25) (layer F.Cu) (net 9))
 (segment (start 70.104 26.416) (end 70.104 22.352) (width 0.25) (layer F.Cu) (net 10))
 (segment (start 67.564 22.352) (end 67.564 26.416) (width 0.25) (layer F.Cu) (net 11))
 (segment (start 65.024 26.416) (end 65.024 22.352) (width 0.25) (layer F.Cu) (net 12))
 (segment (start 62.484 22.352) (end 62.484 26.416) (width 0.25) (layer F.Cu) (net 13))
 (segment (start 85.471 34.671) (end 92.7862 41.9862) (width 0.8) (layer B.Cu) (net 2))
 (segment (start 92.7862 41.9862) (end 92.7862 59.6862) (width 0.8) (layer B.Cu) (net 2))
 (segment (start 92.7862 59.6862) (end 92.79 59.69) (width 0.8) (layer B.Cu) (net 2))
 (segment (start 59.944 26.416) (end 59.944 26.7716) (width 0.8) (layer B.Cu) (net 2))
 (segment (start 59.944 26.7716) (end 61.8744 28.702) (width 0.8) (layer B.Cu) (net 2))
 (segment (start 61.8744 28.702) (end 79.502 28.702) (width 0.8) (layer B.Cu) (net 2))
 (segment (start 79.502 28.702) (end 85.471 34.671) (width 0.8) (layer B.Cu) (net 2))
 (segment (start 92.7862 61.976) (end 92.7862 66.0362) (width 0.8) (layer B.Cu) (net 2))
 (segment (start 92.7862 66.0362) (end 92.79 66.04) (width 0.8) (layer B.Cu) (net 2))
 (segment (start 92.79 59.69) (end 92.7862 59.6938) (width 0.8) (layer B.Cu) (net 2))
 (segment (start 92.7862 59.6938) (end 92.7862 61.976) (width 0.8) (layer B.Cu) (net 2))
 (segment (start 68.66 59.69) (end 92.79 59.69) (width 0.8) (layer B.Cu) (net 2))
 (segment (start 68.66 66.04) (end 68.66 59.69) (width 0.8) (layer B.Cu) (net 2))
 (segment (start 68.66 59.69) (end 50.8 59.69) (width 0.8) (layer B.Cu) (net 2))
 (segment (start 50.8 59.69) (end 44.53 65.96) (width 0.8) (layer B.Cu) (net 2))
 (segment (start 44.53 65.96) (end 44.53 66.04) (width 0.8) (layer B.Cu) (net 2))
 (segment (start 59.944 26.416) (end 59.944 22.352) (width 0.8) (layer F.Cu) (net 2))
 (segment (start 97.409 22.352) (end 85.471 34.29) (width 0.8) (layer B.Cu) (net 2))
 (segment (start 85.471 34.29) (end 85.471 34.671) (width 0.8) (layer B.Cu) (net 2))
 (segment (start 97.409 61.976) (end 92.7862 61.976) (width 0.8) (layer B.Cu) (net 2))
 (segment (start 57.404 22.352) (end 57.404 26.416) (width 0.25) (layer F.Cu) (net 14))
 (segment (start 52.324 41.656) (end 52.324 45.72) (width 0.25) (layer F.Cu) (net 17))
 (segment (start 54.864 45.72) (end 54.864 41.656) (width 0.25) (layer F.Cu) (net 18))
 (segment (start 57.404 41.656) (end 57.404 45.72) (width 0.25) (layer F.Cu) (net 19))
 (segment (start 62.484 41.656) (end 62.484 45.72) (width 0.25) (layer F.Cu) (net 20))
 (segment (start 65.024 45.72) (end 65.024 41.656) (width 0.25) (layer F.Cu) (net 21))
 (segment (start 52.26 52.056) (end 52.26 49.34) (width 0.25) (layer F.Cu) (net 21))
 (segment (start 52.26 49.34) (end 54.102 47.498) (width 0.25) (layer F.Cu) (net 21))
 (segment (start 54.102 47.498) (end 63.246 47.498) (width 0.25) (layer F.Cu) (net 21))
 (segment (start 63.246 47.498) (end 65.024 45.72) (width 0.25) (layer F.Cu) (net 21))
 (segment (start 67.564 45.72) (end 67.564 41.656) (width 0.25) (layer F.Cu) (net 22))
 (segment (start 67.5 52.056) (end 67.564 51.992) (width 0.25) (layer F.Cu) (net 23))
 (segment (start 70.104 41.656) (end 70.104 45.72) (width 0.25) (layer F.Cu) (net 23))
 (segment (start 67.5 52.056) (end 67.5 48.324) (width 0.25) (layer F.Cu) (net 23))
 (segment (start 67.5 48.324) (end 70.104 45.72) (width 0.25) (layer F.Cu) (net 23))
 (segment (start 72.644 45.72) (end 72.644 41.656) (width 0.25) (layer F.Cu) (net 24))
 (segment (start 82.74 52.056) (end 82.74 49.212) (width 0.25) (layer F.Cu) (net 24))
 (segment (start 82.74 49.212) (end 81.026 47.498) (width 0.25) (layer F.Cu) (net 24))
 (segment (start 81.026 47.498) (end 74.422 47.498) (width 0.25) (layer F.Cu) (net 24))
 (segment (start 74.422 47.498) (end 72.644 45.72) (width 0.25) (layer F.Cu) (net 24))
 (segment (start 97.409 32.512) (end 89.154 32.512) (width 0.25) (layer B.Cu) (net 25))
 (segment (start 89.154 32.512) (end 87.376 34.29) (width 0.25) (layer B.Cu) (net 25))
 (segment (start 75.184 41.656) (end 75.184 45.72) (width 0.25) (layer F.Cu) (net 25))
 (segment (start 75.184 41.656) (end 75.184 40.263) (width 0.25) (layer F.Cu) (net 25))
 (segment (start 75.184 40.263) (end 78.871 36.576) (width 0.25) (layer F.Cu) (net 25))
 (segment (start 78.871 36.576) (end 85.09 36.576) (width 0.25) (layer F.Cu) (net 25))
 (segment (start 85.09 36.576) (end 87.376 34.29) (width 0.25) (layer F.Cu) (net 25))
 (segment (start 98.806 35.854) (end 98.806 33.909) (width 0.25) (layer F.Cu) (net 25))
 (segment (start 98.806 33.909) (end 97.409 32.512) (width 0.25) (layer F.Cu) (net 25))
 (via (at 87.376 34.29) (size 1) (layers F.Cu B.Cu) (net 25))
 (segment (start 89.916 37.084) (end 80.903 37.084) (width 0.25) (layer F.Cu) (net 1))
 (segment (start 80.903 37.084) (end 77.724 40.263) (width 0.25) (layer F.Cu) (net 1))
 (segment (start 77.724 40.263) (end 77.724 41.656) (width 0.25) (layer F.Cu) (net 1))
 (segment (start 77.724 45.72) (end 77.724 41.656) (width 0.25) (layer F.Cu) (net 1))
 (segment (start 89.916 37.084) (end 93.726 40.894) (width 0.25) (layer B.Cu) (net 1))
 (segment (start 93.726 40.894) (end 93.726 48.133) (width 0.25) (layer B.Cu) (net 1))
 (segment (start 93.726 48.133) (end 97.409 51.816) (width 0.25) (layer B.Cu) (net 1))
 (segment (start 98.806 48.474) (end 98.806 50.419) (width 0.25) (layer F.Cu) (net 1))
 (segment (start 98.806 50.419) (end 97.409 51.816) (width 0.25) (layer F.Cu) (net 1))
 (via (at 89.916 37.084) (size 1) (layers F.Cu B.Cu) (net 1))
 (segment (start 80.264 41.656) (end 80.264 45.72) (width 0.25) (layer F.Cu) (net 26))
 (segment (start 82.804 45.72) (end 82.804 41.656) (width 0.25) (layer F.Cu) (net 27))
 (segment (start 85.344 41.656) (end 85.344 45.72) (width 0.25) (layer F.Cu) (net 28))
 (segment (start 87.884 45.72) (end 87.884 41.656) (width 0.25) (layer F.Cu) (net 29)))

